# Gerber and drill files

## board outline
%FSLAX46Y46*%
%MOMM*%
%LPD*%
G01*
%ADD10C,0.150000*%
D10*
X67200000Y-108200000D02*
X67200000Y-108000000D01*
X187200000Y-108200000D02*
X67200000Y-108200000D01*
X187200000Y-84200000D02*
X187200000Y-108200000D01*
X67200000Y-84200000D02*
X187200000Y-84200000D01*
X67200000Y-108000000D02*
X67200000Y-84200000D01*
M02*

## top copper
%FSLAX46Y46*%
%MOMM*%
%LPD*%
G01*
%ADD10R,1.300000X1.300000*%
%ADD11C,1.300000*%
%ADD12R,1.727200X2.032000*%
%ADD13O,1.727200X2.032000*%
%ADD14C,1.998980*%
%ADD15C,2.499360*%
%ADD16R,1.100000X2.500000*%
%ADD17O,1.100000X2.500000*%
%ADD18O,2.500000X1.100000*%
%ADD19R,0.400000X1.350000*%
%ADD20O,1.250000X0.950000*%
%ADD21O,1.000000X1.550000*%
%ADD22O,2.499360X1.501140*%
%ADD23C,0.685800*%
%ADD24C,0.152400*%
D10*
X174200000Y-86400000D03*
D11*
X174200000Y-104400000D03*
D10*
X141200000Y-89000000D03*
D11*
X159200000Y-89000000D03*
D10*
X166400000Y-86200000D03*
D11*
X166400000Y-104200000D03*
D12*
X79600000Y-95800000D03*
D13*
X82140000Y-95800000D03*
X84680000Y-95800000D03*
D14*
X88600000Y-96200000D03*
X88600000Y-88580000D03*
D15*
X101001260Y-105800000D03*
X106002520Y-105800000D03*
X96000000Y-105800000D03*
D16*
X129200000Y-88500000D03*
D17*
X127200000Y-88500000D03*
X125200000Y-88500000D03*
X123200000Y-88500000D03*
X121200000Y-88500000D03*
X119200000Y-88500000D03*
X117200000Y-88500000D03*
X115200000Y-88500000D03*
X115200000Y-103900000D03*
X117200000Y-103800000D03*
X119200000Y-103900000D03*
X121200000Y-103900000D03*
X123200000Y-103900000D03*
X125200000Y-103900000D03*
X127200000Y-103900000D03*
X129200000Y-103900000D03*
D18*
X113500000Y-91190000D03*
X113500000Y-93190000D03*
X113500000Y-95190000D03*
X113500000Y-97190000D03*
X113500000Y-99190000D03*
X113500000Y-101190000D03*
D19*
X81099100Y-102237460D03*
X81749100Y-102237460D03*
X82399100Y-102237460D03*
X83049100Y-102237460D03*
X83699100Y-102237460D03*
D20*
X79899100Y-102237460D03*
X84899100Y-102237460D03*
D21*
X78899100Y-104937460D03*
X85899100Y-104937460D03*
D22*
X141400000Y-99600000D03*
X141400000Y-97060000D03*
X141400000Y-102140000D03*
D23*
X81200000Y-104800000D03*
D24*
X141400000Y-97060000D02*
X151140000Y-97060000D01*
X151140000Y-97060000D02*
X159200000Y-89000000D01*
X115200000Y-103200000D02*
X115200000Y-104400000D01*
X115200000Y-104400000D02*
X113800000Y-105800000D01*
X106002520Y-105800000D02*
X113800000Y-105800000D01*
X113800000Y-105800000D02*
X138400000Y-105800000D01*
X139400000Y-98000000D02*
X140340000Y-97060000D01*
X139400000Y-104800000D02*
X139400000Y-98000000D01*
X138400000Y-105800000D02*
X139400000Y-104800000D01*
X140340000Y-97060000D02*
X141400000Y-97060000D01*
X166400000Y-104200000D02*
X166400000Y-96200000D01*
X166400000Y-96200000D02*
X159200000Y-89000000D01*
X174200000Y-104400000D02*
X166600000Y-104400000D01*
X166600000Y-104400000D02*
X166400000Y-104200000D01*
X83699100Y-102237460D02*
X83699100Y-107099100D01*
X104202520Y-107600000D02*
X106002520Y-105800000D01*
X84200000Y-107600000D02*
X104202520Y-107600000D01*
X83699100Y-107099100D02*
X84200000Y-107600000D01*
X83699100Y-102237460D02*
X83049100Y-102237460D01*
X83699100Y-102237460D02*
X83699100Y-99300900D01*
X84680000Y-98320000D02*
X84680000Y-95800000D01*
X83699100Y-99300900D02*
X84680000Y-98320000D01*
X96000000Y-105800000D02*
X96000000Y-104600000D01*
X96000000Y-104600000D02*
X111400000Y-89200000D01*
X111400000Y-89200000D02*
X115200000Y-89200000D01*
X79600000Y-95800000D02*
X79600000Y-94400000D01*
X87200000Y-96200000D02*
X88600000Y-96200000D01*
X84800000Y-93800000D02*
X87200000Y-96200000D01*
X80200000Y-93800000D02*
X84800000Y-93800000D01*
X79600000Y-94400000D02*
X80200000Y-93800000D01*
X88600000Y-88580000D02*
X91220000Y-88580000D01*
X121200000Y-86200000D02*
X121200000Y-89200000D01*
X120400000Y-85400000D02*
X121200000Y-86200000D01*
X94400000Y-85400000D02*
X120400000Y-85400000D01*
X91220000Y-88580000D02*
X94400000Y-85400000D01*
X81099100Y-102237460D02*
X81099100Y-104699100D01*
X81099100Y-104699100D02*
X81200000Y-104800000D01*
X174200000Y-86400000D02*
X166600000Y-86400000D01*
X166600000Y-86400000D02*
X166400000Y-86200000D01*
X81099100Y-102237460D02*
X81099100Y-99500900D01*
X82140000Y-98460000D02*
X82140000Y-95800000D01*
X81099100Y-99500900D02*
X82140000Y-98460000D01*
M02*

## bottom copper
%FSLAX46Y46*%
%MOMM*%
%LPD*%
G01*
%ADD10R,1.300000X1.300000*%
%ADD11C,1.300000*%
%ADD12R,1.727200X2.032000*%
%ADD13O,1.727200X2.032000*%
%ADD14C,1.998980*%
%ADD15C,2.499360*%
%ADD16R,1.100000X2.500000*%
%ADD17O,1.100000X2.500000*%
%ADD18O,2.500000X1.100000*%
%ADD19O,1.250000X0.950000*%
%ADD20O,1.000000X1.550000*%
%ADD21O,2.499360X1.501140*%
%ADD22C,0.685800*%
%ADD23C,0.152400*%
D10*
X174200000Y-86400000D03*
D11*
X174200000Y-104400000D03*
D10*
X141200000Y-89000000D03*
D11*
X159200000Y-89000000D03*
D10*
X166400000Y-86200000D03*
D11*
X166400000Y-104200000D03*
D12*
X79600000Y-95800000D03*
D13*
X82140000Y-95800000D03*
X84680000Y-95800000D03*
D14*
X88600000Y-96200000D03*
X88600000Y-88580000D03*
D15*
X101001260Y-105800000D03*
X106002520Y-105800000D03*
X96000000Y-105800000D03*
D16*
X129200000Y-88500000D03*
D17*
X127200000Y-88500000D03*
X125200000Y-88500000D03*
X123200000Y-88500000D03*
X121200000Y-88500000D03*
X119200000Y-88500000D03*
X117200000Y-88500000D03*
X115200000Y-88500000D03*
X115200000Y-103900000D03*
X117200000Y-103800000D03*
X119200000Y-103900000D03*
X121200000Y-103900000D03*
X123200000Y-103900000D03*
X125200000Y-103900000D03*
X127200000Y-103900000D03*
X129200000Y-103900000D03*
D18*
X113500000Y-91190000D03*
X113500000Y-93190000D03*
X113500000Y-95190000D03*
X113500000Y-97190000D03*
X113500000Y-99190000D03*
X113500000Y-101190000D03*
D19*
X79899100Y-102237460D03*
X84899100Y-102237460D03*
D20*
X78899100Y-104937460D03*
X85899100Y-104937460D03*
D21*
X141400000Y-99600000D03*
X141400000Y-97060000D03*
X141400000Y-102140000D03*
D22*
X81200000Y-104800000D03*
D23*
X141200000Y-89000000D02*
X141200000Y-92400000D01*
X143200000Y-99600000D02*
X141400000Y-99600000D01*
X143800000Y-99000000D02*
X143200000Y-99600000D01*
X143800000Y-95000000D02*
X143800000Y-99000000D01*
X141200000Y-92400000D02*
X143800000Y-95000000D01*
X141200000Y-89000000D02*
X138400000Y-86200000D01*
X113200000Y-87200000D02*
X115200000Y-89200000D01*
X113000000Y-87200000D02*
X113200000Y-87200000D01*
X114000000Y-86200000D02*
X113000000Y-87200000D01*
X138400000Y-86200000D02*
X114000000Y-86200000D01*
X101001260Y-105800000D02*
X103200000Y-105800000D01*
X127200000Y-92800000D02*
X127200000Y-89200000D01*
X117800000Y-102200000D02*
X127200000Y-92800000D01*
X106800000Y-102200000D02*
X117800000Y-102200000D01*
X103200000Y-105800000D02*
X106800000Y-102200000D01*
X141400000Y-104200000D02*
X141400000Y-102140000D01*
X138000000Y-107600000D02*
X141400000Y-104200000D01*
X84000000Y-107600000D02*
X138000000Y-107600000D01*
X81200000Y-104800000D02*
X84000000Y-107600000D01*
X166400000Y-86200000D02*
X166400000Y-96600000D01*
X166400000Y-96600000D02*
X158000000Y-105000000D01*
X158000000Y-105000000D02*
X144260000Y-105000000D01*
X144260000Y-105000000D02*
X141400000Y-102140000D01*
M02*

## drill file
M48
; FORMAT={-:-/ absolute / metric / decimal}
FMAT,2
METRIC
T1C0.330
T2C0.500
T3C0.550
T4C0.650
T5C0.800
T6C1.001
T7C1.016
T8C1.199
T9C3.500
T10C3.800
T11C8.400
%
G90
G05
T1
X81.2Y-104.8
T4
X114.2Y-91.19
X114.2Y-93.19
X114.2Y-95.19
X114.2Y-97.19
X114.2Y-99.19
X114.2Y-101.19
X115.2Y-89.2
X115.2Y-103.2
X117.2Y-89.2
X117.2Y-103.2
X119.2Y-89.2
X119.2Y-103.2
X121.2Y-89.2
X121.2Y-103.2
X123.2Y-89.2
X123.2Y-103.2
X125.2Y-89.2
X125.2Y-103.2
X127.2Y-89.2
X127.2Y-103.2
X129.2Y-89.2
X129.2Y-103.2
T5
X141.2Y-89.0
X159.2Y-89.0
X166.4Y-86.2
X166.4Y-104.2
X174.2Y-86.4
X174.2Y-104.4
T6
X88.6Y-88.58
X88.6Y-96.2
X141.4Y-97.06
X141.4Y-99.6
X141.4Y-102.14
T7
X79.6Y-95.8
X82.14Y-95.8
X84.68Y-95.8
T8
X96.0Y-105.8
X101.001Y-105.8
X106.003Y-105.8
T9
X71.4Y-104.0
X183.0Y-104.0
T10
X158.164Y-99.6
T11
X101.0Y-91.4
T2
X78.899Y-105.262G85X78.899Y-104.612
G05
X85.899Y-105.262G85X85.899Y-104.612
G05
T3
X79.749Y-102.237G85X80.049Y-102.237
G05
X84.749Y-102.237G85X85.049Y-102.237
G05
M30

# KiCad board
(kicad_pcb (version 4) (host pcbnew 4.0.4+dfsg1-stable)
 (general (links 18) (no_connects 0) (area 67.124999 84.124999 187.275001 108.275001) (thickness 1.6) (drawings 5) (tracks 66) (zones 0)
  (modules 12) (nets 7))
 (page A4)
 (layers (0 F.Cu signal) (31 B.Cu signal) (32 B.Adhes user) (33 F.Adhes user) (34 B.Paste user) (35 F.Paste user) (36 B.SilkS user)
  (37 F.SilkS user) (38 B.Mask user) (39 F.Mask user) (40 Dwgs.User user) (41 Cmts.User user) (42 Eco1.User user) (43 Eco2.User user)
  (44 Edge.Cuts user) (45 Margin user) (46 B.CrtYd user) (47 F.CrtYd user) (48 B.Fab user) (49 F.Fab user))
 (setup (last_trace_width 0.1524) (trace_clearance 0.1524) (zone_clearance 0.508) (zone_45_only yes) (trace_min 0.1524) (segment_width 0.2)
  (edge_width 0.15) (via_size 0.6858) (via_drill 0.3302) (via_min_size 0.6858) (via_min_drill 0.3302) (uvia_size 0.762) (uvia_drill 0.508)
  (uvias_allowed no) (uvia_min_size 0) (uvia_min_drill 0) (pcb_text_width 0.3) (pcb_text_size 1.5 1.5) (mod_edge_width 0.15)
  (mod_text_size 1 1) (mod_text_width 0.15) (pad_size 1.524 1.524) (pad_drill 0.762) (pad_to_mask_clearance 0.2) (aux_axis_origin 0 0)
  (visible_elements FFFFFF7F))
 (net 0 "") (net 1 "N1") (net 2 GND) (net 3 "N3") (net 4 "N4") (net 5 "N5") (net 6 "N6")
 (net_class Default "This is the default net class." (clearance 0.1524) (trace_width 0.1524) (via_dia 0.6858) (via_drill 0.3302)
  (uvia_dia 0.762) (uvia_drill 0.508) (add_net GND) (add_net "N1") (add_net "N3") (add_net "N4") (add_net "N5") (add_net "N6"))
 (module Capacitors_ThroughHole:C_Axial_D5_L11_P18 (layer F.Cu) (at 174.2 86.4 270)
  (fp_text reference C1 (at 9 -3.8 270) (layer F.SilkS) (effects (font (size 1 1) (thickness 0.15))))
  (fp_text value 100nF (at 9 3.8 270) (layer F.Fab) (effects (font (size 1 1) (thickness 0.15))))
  (pad 1 thru_hole rect (at 0 0 270) (size 1.3 1.3) (drill 0.8) (layers *.Cu *.Mask F.SilkS) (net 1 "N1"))
  (pad 2 thru_hole circle (at 18 0 270) (size 1.3 1.3) (drill 0.8) (layers *.Cu *.Mask F.SilkS) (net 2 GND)))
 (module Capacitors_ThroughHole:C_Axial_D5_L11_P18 (layer F.Cu) (at 141.2 89)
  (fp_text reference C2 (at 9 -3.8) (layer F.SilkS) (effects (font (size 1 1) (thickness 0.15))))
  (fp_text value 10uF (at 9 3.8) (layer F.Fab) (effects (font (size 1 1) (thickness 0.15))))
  (pad 1 thru_hole rect (at 0 0) (size 1.3 1.3) (drill 0.8) (layers *.Cu *.Mask F.SilkS) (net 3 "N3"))
  (pad 2 thru_hole circle (at 18 0) (size 1.3 1.3) (drill 0.8) (layers *.Cu *.Mask F.SilkS) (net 2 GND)))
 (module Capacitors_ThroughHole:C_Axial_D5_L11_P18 (layer F.Cu) (at 166.4 86.2 270)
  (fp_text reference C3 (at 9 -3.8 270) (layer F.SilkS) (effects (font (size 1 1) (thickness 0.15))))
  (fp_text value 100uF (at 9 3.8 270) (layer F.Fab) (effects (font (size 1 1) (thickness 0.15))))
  (pad 1 thru_hole rect (at 0 0 270) (size 1.3 1.3) (drill 0.8) (layers *.Cu *.Mask F.SilkS) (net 1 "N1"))
  (pad 2 thru_hole circle (at 18 0 270) (size 1.3 1.3) (drill 0.8) (layers *.Cu *.Mask F.SilkS) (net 2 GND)))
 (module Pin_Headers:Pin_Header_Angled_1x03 (layer F.Cu) (at 79.6 95.8 90)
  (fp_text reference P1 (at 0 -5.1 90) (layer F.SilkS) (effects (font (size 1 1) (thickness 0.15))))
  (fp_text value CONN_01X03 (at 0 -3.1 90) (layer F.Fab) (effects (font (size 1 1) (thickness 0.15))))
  (pad 1 thru_hole rect (at 0 0 90) (size 2.032 1.7272) (drill 1.016) (layers *.Cu *.Mask F.SilkS) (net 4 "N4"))
  (pad 2 thru_hole oval (at 0 2.54 90) (size 2.032 1.7272) (drill 1.016) (layers *.Cu *.Mask F.SilkS) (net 1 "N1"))
  (pad 3 thru_hole oval (at 0 5.08 90) (size 2.032 1.7272) (drill 1.016) (layers *.Cu *.Mask F.SilkS) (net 2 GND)))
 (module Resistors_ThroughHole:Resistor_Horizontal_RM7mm (layer F.Cu) (at 88.6 96.2 90)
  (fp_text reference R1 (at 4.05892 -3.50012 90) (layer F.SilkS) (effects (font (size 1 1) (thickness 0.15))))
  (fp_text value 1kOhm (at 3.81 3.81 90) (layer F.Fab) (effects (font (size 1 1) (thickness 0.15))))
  (pad 1 thru_hole circle (at 0 0 90) (size 1.99898 1.99898) (drill 1.00076) (layers *.Cu *.SilkS *.Mask) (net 4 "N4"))
  (pad 2 thru_hole circle (at 7.62 0 90) (size 1.99898 1.99898) (drill 1.00076) (layers *.Cu *.SilkS *.Mask) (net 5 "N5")))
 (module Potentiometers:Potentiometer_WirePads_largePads (layer F.Cu) (at 96 105.8 90)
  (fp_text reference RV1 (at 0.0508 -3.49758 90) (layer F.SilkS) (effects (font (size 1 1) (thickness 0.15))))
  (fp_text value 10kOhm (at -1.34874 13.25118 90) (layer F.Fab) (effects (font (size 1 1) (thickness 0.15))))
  (pad 2 thru_hole circle (at 0 5.00126 90) (size 2.49936 2.49936) (drill 1.19888) (layers *.Cu *.Mask F.SilkS) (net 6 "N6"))
  (pad 3 thru_hole circle (at 0 10.00252 90) (size 2.49936 2.49936) (drill 1.19888) (layers *.Cu *.Mask F.SilkS) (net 2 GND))
  (pad 1 thru_hole circle (at 0 0 90) (size 2.49936 2.49936) (drill 1.19888) (layers *.Cu *.Mask F.SilkS) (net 3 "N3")))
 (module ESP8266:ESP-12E (layer F.Cu) (at 129.2 89.2 270)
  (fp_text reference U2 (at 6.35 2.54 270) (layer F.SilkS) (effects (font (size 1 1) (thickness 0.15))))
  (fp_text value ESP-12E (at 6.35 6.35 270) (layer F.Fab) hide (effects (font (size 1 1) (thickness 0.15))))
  (pad 1 thru_hole rect (at 0 0 270) (size 2.5 1.1) (drill 0.65 (offset -0.7 0)) (layers *.Cu *.Mask F.SilkS))
  (pad 2 thru_hole oval (at 0 2 270) (size 2.5 1.1) (drill 0.65 (offset -0.7 0)) (layers *.Cu *.Mask F.SilkS) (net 6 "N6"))
  (pad 3 thru_hole oval (at 0 4 270) (size 2.5 1.1) (drill 0.65 (offset -0.7 0)) (layers *.Cu *.Mask F.SilkS))
  (pad 4 thru_hole oval (at 0 6 270) (size 2.5 1.1) (drill 0.65 (offset -0.7 0)) (layers *.Cu *.Mask F.SilkS))
  (pad 5 thru_hole oval (at 0 8 270) (size 2.5 1.1) (drill 0.65 (offset -0.7 0)) (layers *.Cu *.Mask F.SilkS) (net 5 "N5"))
  (pad 6 thru_hole oval (at 0 10 270) (size 2.5 1.1) (drill 0.65 (offset -0.7 0)) (layers *.Cu *.Mask F.SilkS))
  (pad 7 thru_hole oval (at 0 12 270) (size 2.5 1.1) (drill 0.65 (offset -0.7 0)) (layers *.Cu *.Mask F.SilkS))
  (pad 8 thru_hole oval (at 0 14 270) (size 2.5 1.1) (drill 0.65 (offset -0.7 0)) (layers *.Cu *.Mask F.SilkS) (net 3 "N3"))
  (pad 9 thru_hole oval (at 14 14 270) (size 2.5 1.1) (drill 0.65 (offset 0.7 0)) (layers *.Cu *.Mask F.SilkS) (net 2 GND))
  (pad 10 thru_hole oval (at 14 12 270) (size 2.5 1.1) (drill 0.65 (offset 0.6 0)) (layers *.Cu *.Mask F.SilkS))
  (pad 11 thru_hole oval (at 14 10 270) (size 2.5 1.1) (drill 0.65 (offset 0.7 0)) (layers *.Cu *.Mask F.SilkS))
  (pad 12 thru_hole oval (at 14 8 270) (size 2.5 1.1) (drill 0.65 (offset 0.7 0)) (layers *.Cu *.Mask F.SilkS))
  (pad 13 thru_hole oval (at 14 6 270) (size 2.5 1.1) (drill 0.65 (offset 0.7 0)) (layers *.Cu *.Mask F.SilkS))
  (pad 14 thru_hole oval (at 14 4 270) (size 2.5 1.1) (drill 0.65 (offset 0.7 0)) (layers *.Cu *.Mask F.SilkS))
  (pad 15 thru_hole oval (at 14 2 270) (size 2.5 1.1) (drill 0.65 (offset 0.7 0)) (layers *.Cu *.Mask F.SilkS))
  (pad 16 thru_hole oval (at 14 0 270) (size 2.5 1.1) (drill 0.65 (offset 0.7 0)) (layers *.Cu *.Mask F.SilkS))
  (pad 17 thru_hole oval (at 1.99 15) (size 2.5 1.1) (drill 0.65 (offset -0.7 0)) (layers *.Cu *.Mask F.SilkS))
  (pad 18 thru_hole oval (at 3.99 15) (size 2.5 1.1) (drill 0.65 (offset -0.7 0)) (layers *.Cu *.Mask F.SilkS))
  (pad 19 thru_hole oval (at 5.99 15) (size 2.5 1.1) (drill 0.65 (offset -0.7 0)) (layers *.Cu *.Mask F.SilkS))
  (pad 20 thru_hole oval (at 7.99 15) (size 2.5 1.1) (drill 0.65 (offset -0.7 0)) (layers *.Cu *.Mask F.SilkS))
  (pad 21 thru_hole oval (at 9.99 15) (size 2.5 1.1) (drill 0.65 (offset -0.7 0)) (layers *.Cu *.Mask F.SilkS))
  (pad 22 thru_hole oval (at 11.99 15) (size 2.5 1.1) (drill 0.65 (offset -0.7 0)) (layers *.Cu *.Mask F.SilkS)))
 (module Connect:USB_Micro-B (layer F.Cu) (at 82.4 103.8)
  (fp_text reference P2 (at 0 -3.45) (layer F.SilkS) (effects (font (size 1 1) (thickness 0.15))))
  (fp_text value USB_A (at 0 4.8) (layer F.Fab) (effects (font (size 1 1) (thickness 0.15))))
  (pad 1 smd rect (at -1.3009 -1.56254 90) (size 1.35 0.4) (layers F.Cu F.Paste F.Mask) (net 1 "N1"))
  (pad 2 smd rect (at -0.6509 -1.56254 90) (size 1.35 0.4) (layers F.Cu F.Paste F.Mask))
  (pad 3 smd rect (at -0.0009 -1.56254 90) (size 1.35 0.4) (layers F.Cu F.Paste F.Mask))
  (pad 4 smd rect (at 0.6491 -1.56254 90) (size 1.35 0.4) (layers F.Cu F.Paste F.Mask) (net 2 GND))
  (pad 5 smd rect (at 1.2991 -1.56254 90) (size 1.35 0.4) (layers F.Cu F.Paste F.Mask) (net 2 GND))
  (pad 6 thru_hole oval (at -2.5009 -1.56254 90) (size 0.95 1.25) (drill oval 0.55 0.85) (layers *.Cu *.Mask F.SilkS))
  (pad 6 thru_hole oval (at 2.4991 -1.56254 90) (size 0.95 1.25) (drill oval 0.55 0.85) (layers *.Cu *.Mask F.SilkS))
  (pad 6 thru_hole oval (at -3.5009 1.13746 90) (size 1.55 1) (drill oval 1.15 0.5) (layers *.Cu *.Mask F.SilkS))
  (pad 6 thru_hole oval (at 3.4991 1.13746 90) (size 1.55 1) (drill oval 1.15 0.5) (layers *.Cu *.Mask F.SilkS)))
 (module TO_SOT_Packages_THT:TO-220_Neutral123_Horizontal (layer F.Cu) (at 141.4 99.6 270)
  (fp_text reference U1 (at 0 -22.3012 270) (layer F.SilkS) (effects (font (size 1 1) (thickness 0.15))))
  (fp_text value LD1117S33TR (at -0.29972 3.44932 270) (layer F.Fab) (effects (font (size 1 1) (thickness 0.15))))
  (pad 2 thru_hole oval (at 0 0) (size 2.49936 1.50114) (drill 1.00076) (layers *.Cu *.Mask F.SilkS) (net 3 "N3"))
  (pad 1 thru_hole oval (at -2.54 0) (size 2.49936 1.50114) (drill 1.00076) (layers *.Cu *.Mask F.SilkS) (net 2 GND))
  (pad 3 thru_hole oval (at 2.54 0) (size 2.49936 1.50114) (drill 1.00076) (layers *.Cu *.Mask F.SilkS) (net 1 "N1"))
  (pad "" np_thru_hole circle (at 0 -16.764) (size 3.79984 3.79984) (drill 3.79984) (layers *.Cu *.Mask F.SilkS)))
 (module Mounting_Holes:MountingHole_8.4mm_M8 (layer F.Cu) (at 101 91.4)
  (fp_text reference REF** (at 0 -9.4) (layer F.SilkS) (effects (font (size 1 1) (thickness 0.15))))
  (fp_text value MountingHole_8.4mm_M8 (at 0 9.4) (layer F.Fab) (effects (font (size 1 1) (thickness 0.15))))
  (pad 1 np_thru_hole circle (at 0 0) (size 8.4 8.4) (drill 8.4) (layers *.Cu *.Mask F.SilkS)))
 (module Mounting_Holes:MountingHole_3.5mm (layer F.Cu) (at 71.4 104)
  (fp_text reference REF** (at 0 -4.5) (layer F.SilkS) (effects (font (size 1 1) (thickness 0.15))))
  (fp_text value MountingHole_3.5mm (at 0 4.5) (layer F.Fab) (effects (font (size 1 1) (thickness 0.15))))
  (pad 1 np_thru_hole circle (at 0 0) (size 3.5 3.5) (drill 3.5) (layers *.Cu *.Mask F.SilkS)))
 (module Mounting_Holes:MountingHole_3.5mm (layer F.Cu) (at 183 104)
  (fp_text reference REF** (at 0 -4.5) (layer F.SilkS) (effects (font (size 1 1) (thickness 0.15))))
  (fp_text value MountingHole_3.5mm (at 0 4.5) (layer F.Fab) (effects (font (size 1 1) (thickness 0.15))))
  (pad 1 np_thru_hole circle (at 0 0) (size 3.5 3.5) (drill 3.5) (layers *.Cu *.Mask F.SilkS)))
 (gr_line (start 67.2 108.2) (end 67.2 108) (angle 90) (layer Edge.Cuts) (width 0.15))
 (gr_line (start 187.2 108.2) (end 67.2 108.2) (angle 90) (layer Edge.Cuts) (width 0.15))
 (gr_line (start 187.2 84.2) (end 187.2 108.2) (angle 90) (layer Edge.Cuts) (width 0.15))
 (gr_line (start 67.2 84.2) (end 187.2 84.2) (angle 90) (layer Edge.Cuts) (width 0.15))
 (gr_line (start 67.2 108) (end 67.2 84.2) (angle 90) (layer Edge.Cuts) (width 0.15))
 (segment (start 141.4 97.06) (end 151.14 97.06) (width 0.1524) (layer F.Cu) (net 2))
 (segment (start 151.14 97.06) (end 159.2 89) (width 0.1524) (layer F.Cu) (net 2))
 (segment (start 115.2 103.2) (end 115.2 104.4) (width 0.1524) (layer F.Cu) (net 2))
 (segment (start 115.2 104.4) (end 113.8 105.8) (width 0.1524) (layer F.Cu) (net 2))
 (segment (start 106.00252 105.8) (end 113.8 105.8) (width 0.1524) (layer F.Cu) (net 2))
 (segment (start 113.8 105.8) (end 138.4 105.8) (width 0.1524) (layer F.Cu) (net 2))
 (segment (start 139.4 98) (end 140.34 97.06) (width 0.1524) (layer F.Cu) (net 2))
 (segment (start 139.4 104.8) (end 139.4 98) (width 0.1524) (layer F.Cu) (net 2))
 (segment (start 138.4 105.8) (end 139.4 104.8) (width 0.1524) (layer F.Cu) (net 2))
 (segment (start 140.34 97.06) (end 141.4 97.06) (width 0.1524) (layer F.Cu) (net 2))
 (segment (start 166.4 104.2) (end 166.4 96.2) (width 0.1524) (layer F.Cu) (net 2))
 (segment (start 166.4 96.2) (end 159.2 89) (width 0.1524) (layer F.Cu) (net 2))
 (segment (start 174.2 104.4) (end 166.6 104.4) (width 0.1524) (layer F.Cu) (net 2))
 (segment (start 166.6 104.4) (end 166.4 104.2) (width 0.1524) (layer F.Cu) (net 2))
 (segment (start 83.6991 102.23746) (end 83.6991 107.0991) (width 0.1524) (layer F.Cu) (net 2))
 (segment (start 104.20252 107.6) (end 106.00252 105.8) (width 0.1524) (layer F.Cu) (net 2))
 (segment (start 84.2 107.6) (end 104.20252 107.6) (width 0.1524) (layer F.Cu) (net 2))
 (segment (start 83.6991 107.0991) (end 84.2 107.6) (width 0.1524) (layer F.Cu) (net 2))
 (segment (start 83.6991 102.23746) (end 83.0491 102.23746) (width 0.1524) (layer F.Cu) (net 2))
 (segment (start 83.6991 102.23746) (end 83.6991 99.3009) (width 0.1524) (layer F.Cu) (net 2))
 (segment (start 84.68 98.32) (end 84.68 95.8) (width 0.1524) (layer F.Cu) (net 2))
 (segment (start 83.6991 99.3009) (end 84.68 98.32) (width 0.1524) (layer F.Cu) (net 2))
 (segment (start 141.2 89) (end 141.2 92.4) (width 0.1524) (layer B.Cu) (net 3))
 (segment (start 143.2 99.6) (end 141.4 99.6) (width 0.1524) (layer B.Cu) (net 3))
 (segment (start 143.8 99) (end 143.2 99.6) (width 0.1524) (layer B.Cu) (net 3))
 (segment (start 143.8 95) (end 143.8 99) (width 0.1524) (layer B.Cu) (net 3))
 (segment (start 141.2 92.4) (end 143.8 95) (width 0.1524) (layer B.Cu) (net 3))
 (segment (start 141.2 89) (end 138.4 86.2) (width 0.1524) (layer B.Cu) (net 3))
 (segment (start 113.2 87.2) (end 115.2 89.2) (width 0.1524) (layer B.Cu) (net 3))
 (segment (start 113 87.2) (end 113.2 87.2) (width 0.1524) (layer B.Cu) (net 3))
 (segment (start 114 86.2) (end 113 87.2) (width 0.1524) (layer B.Cu) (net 3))
 (segment (start 138.4 86.2) (end 114 86.2) (width 0.1524) (layer B.Cu) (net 3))
 (segment (start 96 105.8) (end 96 104.6) (width 0.1524) (layer F.Cu) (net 3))
 (segment (start 96 104.6) (end 111.4 89.2) (width 0.1524) (layer F.Cu) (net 3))
 (segment (start 111.4 89.2) (end 115.2 89.2) (width 0.1524) (layer F.Cu) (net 3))
 (segment (start 79.6 95.8) (end 79.6 94.4) (width 0.1524) (layer F.Cu) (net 4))
 (segment (start 87.2 96.2) (end 88.6 96.2) (width 0.1524) (layer F.Cu) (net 4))
 (segment (start 84.8 93.8) (end 87.2 96.2) (width 0.1524) (layer F.Cu) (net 4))
 (segment (start 80.2 93.8) (end 84.8 93.8) (width 0.1524) (layer F.Cu) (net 4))
 (segment (start 79.6 94.4) (end 80.2 93.8) (width 0.1524) (layer F.Cu) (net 4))
 (segment (start 88.6 88.58) (end 91.22 88.58) (width 0.1524) (layer F.Cu) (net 5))
 (segment (start 121.2 86.2) (end 121.2 89.2) (width 0.1524) (layer F.Cu) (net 5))
 (segment (start 120.4 85.4) (end 121.2 86.2) (width 0.1524) (layer F.Cu) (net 5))
 (segment (start 94.4 85.4) (end 120.4 85.4) (width 0.1524) (layer F.Cu) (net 5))
 (segment (start 91.22 88.58) (end 94.4 85.4) (width 0.1524) (layer F.Cu) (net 5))
 (segment (start 101.00126 105.8) (end 103.2 105.8) (width 0.1524) (layer B.Cu) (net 6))
 (segment (start 127.2 92.8) (end 127.2 89.2) (width 0.1524) (layer B.Cu) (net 6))
 (segment (start 117.8 102.2) (end 127.2 92.8) (width 0.1524) (layer B.Cu) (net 6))
 (segment (start 106.8 102.2) (end 117.8 102.2) (width 0.1524) (layer B.Cu) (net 6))
 (segment (start 103.2 105.8) (end 106.8 102.2) (width 0.1524) (layer B.Cu) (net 6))
 (segment (start 81.0991 102.23746) (end 81.0991 104.6991) (width 0.1524) (layer F.Cu) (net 1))
 (segment (start 141.4 104.2) (end 141.4 102.14) (width 0.1524) (layer B.Cu) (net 1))
 (segment (start 138 107.6) (end 141.4 104.2) (width 0.1524) (layer B.Cu) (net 1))
 (segment (start 84 107.6) (end 138 107.6) (width 0.1524) (layer B.Cu) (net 1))
 (segment (start 81.2 104.8) (end 84 107.6) (width 0.1524) (layer B.Cu) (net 1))
 (via (at 81.2 104.8) (size 0.6858) (drill 0.3302) (layers F.Cu B.Cu) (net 1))
 (segment (start 81.0991 104.6991) (end 81.2 104.8) (width 0.1524) (layer F.Cu) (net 1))
 (segment (start 166.4 86.2) (end 166.4 96.6) (width 0.1524) (layer B.Cu) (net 1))
 (segment (start 166.4 96.6) (end 158 105) (width 0.1524) (layer B.Cu) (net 1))
 (segment (start 158 105) (end 144.26 105) (width 0.1524) (layer B.Cu) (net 1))
 (segment (start 144.26 105) (end 141.4 102.14) (width 0.1524) (layer B.Cu) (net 1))
 (segment (start 174.2 86.4) (end 166.6 86.4) (width 0.1524) (layer F.Cu) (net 1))
 (segment (start 166.6 86.4) (end 166.4 86.2) (width 0.1524) (layer F.Cu) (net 1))
 (segment (start 81.0991 102.23746) (end 81.0991 99.5009) (width 0.1524) (layer F.Cu) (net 1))
 (segment (start 82.14 98.46) (end 82.14 95.8) (width 0.1524) (layer F.Cu) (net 1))
 (segment (start 81.0991 99.5009) (end 82.14 98.46) (width 0.1524) (layer F.Cu) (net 1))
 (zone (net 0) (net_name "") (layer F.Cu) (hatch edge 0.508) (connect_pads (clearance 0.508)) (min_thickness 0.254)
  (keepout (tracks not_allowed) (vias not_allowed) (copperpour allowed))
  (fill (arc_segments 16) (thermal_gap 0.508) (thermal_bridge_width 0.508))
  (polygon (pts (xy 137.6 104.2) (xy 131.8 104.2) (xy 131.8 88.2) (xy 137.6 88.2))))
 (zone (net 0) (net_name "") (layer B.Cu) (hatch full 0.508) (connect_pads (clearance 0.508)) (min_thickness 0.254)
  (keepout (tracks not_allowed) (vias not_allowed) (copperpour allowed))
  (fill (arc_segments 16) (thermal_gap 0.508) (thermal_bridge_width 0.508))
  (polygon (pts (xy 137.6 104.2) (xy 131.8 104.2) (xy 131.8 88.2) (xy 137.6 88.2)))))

